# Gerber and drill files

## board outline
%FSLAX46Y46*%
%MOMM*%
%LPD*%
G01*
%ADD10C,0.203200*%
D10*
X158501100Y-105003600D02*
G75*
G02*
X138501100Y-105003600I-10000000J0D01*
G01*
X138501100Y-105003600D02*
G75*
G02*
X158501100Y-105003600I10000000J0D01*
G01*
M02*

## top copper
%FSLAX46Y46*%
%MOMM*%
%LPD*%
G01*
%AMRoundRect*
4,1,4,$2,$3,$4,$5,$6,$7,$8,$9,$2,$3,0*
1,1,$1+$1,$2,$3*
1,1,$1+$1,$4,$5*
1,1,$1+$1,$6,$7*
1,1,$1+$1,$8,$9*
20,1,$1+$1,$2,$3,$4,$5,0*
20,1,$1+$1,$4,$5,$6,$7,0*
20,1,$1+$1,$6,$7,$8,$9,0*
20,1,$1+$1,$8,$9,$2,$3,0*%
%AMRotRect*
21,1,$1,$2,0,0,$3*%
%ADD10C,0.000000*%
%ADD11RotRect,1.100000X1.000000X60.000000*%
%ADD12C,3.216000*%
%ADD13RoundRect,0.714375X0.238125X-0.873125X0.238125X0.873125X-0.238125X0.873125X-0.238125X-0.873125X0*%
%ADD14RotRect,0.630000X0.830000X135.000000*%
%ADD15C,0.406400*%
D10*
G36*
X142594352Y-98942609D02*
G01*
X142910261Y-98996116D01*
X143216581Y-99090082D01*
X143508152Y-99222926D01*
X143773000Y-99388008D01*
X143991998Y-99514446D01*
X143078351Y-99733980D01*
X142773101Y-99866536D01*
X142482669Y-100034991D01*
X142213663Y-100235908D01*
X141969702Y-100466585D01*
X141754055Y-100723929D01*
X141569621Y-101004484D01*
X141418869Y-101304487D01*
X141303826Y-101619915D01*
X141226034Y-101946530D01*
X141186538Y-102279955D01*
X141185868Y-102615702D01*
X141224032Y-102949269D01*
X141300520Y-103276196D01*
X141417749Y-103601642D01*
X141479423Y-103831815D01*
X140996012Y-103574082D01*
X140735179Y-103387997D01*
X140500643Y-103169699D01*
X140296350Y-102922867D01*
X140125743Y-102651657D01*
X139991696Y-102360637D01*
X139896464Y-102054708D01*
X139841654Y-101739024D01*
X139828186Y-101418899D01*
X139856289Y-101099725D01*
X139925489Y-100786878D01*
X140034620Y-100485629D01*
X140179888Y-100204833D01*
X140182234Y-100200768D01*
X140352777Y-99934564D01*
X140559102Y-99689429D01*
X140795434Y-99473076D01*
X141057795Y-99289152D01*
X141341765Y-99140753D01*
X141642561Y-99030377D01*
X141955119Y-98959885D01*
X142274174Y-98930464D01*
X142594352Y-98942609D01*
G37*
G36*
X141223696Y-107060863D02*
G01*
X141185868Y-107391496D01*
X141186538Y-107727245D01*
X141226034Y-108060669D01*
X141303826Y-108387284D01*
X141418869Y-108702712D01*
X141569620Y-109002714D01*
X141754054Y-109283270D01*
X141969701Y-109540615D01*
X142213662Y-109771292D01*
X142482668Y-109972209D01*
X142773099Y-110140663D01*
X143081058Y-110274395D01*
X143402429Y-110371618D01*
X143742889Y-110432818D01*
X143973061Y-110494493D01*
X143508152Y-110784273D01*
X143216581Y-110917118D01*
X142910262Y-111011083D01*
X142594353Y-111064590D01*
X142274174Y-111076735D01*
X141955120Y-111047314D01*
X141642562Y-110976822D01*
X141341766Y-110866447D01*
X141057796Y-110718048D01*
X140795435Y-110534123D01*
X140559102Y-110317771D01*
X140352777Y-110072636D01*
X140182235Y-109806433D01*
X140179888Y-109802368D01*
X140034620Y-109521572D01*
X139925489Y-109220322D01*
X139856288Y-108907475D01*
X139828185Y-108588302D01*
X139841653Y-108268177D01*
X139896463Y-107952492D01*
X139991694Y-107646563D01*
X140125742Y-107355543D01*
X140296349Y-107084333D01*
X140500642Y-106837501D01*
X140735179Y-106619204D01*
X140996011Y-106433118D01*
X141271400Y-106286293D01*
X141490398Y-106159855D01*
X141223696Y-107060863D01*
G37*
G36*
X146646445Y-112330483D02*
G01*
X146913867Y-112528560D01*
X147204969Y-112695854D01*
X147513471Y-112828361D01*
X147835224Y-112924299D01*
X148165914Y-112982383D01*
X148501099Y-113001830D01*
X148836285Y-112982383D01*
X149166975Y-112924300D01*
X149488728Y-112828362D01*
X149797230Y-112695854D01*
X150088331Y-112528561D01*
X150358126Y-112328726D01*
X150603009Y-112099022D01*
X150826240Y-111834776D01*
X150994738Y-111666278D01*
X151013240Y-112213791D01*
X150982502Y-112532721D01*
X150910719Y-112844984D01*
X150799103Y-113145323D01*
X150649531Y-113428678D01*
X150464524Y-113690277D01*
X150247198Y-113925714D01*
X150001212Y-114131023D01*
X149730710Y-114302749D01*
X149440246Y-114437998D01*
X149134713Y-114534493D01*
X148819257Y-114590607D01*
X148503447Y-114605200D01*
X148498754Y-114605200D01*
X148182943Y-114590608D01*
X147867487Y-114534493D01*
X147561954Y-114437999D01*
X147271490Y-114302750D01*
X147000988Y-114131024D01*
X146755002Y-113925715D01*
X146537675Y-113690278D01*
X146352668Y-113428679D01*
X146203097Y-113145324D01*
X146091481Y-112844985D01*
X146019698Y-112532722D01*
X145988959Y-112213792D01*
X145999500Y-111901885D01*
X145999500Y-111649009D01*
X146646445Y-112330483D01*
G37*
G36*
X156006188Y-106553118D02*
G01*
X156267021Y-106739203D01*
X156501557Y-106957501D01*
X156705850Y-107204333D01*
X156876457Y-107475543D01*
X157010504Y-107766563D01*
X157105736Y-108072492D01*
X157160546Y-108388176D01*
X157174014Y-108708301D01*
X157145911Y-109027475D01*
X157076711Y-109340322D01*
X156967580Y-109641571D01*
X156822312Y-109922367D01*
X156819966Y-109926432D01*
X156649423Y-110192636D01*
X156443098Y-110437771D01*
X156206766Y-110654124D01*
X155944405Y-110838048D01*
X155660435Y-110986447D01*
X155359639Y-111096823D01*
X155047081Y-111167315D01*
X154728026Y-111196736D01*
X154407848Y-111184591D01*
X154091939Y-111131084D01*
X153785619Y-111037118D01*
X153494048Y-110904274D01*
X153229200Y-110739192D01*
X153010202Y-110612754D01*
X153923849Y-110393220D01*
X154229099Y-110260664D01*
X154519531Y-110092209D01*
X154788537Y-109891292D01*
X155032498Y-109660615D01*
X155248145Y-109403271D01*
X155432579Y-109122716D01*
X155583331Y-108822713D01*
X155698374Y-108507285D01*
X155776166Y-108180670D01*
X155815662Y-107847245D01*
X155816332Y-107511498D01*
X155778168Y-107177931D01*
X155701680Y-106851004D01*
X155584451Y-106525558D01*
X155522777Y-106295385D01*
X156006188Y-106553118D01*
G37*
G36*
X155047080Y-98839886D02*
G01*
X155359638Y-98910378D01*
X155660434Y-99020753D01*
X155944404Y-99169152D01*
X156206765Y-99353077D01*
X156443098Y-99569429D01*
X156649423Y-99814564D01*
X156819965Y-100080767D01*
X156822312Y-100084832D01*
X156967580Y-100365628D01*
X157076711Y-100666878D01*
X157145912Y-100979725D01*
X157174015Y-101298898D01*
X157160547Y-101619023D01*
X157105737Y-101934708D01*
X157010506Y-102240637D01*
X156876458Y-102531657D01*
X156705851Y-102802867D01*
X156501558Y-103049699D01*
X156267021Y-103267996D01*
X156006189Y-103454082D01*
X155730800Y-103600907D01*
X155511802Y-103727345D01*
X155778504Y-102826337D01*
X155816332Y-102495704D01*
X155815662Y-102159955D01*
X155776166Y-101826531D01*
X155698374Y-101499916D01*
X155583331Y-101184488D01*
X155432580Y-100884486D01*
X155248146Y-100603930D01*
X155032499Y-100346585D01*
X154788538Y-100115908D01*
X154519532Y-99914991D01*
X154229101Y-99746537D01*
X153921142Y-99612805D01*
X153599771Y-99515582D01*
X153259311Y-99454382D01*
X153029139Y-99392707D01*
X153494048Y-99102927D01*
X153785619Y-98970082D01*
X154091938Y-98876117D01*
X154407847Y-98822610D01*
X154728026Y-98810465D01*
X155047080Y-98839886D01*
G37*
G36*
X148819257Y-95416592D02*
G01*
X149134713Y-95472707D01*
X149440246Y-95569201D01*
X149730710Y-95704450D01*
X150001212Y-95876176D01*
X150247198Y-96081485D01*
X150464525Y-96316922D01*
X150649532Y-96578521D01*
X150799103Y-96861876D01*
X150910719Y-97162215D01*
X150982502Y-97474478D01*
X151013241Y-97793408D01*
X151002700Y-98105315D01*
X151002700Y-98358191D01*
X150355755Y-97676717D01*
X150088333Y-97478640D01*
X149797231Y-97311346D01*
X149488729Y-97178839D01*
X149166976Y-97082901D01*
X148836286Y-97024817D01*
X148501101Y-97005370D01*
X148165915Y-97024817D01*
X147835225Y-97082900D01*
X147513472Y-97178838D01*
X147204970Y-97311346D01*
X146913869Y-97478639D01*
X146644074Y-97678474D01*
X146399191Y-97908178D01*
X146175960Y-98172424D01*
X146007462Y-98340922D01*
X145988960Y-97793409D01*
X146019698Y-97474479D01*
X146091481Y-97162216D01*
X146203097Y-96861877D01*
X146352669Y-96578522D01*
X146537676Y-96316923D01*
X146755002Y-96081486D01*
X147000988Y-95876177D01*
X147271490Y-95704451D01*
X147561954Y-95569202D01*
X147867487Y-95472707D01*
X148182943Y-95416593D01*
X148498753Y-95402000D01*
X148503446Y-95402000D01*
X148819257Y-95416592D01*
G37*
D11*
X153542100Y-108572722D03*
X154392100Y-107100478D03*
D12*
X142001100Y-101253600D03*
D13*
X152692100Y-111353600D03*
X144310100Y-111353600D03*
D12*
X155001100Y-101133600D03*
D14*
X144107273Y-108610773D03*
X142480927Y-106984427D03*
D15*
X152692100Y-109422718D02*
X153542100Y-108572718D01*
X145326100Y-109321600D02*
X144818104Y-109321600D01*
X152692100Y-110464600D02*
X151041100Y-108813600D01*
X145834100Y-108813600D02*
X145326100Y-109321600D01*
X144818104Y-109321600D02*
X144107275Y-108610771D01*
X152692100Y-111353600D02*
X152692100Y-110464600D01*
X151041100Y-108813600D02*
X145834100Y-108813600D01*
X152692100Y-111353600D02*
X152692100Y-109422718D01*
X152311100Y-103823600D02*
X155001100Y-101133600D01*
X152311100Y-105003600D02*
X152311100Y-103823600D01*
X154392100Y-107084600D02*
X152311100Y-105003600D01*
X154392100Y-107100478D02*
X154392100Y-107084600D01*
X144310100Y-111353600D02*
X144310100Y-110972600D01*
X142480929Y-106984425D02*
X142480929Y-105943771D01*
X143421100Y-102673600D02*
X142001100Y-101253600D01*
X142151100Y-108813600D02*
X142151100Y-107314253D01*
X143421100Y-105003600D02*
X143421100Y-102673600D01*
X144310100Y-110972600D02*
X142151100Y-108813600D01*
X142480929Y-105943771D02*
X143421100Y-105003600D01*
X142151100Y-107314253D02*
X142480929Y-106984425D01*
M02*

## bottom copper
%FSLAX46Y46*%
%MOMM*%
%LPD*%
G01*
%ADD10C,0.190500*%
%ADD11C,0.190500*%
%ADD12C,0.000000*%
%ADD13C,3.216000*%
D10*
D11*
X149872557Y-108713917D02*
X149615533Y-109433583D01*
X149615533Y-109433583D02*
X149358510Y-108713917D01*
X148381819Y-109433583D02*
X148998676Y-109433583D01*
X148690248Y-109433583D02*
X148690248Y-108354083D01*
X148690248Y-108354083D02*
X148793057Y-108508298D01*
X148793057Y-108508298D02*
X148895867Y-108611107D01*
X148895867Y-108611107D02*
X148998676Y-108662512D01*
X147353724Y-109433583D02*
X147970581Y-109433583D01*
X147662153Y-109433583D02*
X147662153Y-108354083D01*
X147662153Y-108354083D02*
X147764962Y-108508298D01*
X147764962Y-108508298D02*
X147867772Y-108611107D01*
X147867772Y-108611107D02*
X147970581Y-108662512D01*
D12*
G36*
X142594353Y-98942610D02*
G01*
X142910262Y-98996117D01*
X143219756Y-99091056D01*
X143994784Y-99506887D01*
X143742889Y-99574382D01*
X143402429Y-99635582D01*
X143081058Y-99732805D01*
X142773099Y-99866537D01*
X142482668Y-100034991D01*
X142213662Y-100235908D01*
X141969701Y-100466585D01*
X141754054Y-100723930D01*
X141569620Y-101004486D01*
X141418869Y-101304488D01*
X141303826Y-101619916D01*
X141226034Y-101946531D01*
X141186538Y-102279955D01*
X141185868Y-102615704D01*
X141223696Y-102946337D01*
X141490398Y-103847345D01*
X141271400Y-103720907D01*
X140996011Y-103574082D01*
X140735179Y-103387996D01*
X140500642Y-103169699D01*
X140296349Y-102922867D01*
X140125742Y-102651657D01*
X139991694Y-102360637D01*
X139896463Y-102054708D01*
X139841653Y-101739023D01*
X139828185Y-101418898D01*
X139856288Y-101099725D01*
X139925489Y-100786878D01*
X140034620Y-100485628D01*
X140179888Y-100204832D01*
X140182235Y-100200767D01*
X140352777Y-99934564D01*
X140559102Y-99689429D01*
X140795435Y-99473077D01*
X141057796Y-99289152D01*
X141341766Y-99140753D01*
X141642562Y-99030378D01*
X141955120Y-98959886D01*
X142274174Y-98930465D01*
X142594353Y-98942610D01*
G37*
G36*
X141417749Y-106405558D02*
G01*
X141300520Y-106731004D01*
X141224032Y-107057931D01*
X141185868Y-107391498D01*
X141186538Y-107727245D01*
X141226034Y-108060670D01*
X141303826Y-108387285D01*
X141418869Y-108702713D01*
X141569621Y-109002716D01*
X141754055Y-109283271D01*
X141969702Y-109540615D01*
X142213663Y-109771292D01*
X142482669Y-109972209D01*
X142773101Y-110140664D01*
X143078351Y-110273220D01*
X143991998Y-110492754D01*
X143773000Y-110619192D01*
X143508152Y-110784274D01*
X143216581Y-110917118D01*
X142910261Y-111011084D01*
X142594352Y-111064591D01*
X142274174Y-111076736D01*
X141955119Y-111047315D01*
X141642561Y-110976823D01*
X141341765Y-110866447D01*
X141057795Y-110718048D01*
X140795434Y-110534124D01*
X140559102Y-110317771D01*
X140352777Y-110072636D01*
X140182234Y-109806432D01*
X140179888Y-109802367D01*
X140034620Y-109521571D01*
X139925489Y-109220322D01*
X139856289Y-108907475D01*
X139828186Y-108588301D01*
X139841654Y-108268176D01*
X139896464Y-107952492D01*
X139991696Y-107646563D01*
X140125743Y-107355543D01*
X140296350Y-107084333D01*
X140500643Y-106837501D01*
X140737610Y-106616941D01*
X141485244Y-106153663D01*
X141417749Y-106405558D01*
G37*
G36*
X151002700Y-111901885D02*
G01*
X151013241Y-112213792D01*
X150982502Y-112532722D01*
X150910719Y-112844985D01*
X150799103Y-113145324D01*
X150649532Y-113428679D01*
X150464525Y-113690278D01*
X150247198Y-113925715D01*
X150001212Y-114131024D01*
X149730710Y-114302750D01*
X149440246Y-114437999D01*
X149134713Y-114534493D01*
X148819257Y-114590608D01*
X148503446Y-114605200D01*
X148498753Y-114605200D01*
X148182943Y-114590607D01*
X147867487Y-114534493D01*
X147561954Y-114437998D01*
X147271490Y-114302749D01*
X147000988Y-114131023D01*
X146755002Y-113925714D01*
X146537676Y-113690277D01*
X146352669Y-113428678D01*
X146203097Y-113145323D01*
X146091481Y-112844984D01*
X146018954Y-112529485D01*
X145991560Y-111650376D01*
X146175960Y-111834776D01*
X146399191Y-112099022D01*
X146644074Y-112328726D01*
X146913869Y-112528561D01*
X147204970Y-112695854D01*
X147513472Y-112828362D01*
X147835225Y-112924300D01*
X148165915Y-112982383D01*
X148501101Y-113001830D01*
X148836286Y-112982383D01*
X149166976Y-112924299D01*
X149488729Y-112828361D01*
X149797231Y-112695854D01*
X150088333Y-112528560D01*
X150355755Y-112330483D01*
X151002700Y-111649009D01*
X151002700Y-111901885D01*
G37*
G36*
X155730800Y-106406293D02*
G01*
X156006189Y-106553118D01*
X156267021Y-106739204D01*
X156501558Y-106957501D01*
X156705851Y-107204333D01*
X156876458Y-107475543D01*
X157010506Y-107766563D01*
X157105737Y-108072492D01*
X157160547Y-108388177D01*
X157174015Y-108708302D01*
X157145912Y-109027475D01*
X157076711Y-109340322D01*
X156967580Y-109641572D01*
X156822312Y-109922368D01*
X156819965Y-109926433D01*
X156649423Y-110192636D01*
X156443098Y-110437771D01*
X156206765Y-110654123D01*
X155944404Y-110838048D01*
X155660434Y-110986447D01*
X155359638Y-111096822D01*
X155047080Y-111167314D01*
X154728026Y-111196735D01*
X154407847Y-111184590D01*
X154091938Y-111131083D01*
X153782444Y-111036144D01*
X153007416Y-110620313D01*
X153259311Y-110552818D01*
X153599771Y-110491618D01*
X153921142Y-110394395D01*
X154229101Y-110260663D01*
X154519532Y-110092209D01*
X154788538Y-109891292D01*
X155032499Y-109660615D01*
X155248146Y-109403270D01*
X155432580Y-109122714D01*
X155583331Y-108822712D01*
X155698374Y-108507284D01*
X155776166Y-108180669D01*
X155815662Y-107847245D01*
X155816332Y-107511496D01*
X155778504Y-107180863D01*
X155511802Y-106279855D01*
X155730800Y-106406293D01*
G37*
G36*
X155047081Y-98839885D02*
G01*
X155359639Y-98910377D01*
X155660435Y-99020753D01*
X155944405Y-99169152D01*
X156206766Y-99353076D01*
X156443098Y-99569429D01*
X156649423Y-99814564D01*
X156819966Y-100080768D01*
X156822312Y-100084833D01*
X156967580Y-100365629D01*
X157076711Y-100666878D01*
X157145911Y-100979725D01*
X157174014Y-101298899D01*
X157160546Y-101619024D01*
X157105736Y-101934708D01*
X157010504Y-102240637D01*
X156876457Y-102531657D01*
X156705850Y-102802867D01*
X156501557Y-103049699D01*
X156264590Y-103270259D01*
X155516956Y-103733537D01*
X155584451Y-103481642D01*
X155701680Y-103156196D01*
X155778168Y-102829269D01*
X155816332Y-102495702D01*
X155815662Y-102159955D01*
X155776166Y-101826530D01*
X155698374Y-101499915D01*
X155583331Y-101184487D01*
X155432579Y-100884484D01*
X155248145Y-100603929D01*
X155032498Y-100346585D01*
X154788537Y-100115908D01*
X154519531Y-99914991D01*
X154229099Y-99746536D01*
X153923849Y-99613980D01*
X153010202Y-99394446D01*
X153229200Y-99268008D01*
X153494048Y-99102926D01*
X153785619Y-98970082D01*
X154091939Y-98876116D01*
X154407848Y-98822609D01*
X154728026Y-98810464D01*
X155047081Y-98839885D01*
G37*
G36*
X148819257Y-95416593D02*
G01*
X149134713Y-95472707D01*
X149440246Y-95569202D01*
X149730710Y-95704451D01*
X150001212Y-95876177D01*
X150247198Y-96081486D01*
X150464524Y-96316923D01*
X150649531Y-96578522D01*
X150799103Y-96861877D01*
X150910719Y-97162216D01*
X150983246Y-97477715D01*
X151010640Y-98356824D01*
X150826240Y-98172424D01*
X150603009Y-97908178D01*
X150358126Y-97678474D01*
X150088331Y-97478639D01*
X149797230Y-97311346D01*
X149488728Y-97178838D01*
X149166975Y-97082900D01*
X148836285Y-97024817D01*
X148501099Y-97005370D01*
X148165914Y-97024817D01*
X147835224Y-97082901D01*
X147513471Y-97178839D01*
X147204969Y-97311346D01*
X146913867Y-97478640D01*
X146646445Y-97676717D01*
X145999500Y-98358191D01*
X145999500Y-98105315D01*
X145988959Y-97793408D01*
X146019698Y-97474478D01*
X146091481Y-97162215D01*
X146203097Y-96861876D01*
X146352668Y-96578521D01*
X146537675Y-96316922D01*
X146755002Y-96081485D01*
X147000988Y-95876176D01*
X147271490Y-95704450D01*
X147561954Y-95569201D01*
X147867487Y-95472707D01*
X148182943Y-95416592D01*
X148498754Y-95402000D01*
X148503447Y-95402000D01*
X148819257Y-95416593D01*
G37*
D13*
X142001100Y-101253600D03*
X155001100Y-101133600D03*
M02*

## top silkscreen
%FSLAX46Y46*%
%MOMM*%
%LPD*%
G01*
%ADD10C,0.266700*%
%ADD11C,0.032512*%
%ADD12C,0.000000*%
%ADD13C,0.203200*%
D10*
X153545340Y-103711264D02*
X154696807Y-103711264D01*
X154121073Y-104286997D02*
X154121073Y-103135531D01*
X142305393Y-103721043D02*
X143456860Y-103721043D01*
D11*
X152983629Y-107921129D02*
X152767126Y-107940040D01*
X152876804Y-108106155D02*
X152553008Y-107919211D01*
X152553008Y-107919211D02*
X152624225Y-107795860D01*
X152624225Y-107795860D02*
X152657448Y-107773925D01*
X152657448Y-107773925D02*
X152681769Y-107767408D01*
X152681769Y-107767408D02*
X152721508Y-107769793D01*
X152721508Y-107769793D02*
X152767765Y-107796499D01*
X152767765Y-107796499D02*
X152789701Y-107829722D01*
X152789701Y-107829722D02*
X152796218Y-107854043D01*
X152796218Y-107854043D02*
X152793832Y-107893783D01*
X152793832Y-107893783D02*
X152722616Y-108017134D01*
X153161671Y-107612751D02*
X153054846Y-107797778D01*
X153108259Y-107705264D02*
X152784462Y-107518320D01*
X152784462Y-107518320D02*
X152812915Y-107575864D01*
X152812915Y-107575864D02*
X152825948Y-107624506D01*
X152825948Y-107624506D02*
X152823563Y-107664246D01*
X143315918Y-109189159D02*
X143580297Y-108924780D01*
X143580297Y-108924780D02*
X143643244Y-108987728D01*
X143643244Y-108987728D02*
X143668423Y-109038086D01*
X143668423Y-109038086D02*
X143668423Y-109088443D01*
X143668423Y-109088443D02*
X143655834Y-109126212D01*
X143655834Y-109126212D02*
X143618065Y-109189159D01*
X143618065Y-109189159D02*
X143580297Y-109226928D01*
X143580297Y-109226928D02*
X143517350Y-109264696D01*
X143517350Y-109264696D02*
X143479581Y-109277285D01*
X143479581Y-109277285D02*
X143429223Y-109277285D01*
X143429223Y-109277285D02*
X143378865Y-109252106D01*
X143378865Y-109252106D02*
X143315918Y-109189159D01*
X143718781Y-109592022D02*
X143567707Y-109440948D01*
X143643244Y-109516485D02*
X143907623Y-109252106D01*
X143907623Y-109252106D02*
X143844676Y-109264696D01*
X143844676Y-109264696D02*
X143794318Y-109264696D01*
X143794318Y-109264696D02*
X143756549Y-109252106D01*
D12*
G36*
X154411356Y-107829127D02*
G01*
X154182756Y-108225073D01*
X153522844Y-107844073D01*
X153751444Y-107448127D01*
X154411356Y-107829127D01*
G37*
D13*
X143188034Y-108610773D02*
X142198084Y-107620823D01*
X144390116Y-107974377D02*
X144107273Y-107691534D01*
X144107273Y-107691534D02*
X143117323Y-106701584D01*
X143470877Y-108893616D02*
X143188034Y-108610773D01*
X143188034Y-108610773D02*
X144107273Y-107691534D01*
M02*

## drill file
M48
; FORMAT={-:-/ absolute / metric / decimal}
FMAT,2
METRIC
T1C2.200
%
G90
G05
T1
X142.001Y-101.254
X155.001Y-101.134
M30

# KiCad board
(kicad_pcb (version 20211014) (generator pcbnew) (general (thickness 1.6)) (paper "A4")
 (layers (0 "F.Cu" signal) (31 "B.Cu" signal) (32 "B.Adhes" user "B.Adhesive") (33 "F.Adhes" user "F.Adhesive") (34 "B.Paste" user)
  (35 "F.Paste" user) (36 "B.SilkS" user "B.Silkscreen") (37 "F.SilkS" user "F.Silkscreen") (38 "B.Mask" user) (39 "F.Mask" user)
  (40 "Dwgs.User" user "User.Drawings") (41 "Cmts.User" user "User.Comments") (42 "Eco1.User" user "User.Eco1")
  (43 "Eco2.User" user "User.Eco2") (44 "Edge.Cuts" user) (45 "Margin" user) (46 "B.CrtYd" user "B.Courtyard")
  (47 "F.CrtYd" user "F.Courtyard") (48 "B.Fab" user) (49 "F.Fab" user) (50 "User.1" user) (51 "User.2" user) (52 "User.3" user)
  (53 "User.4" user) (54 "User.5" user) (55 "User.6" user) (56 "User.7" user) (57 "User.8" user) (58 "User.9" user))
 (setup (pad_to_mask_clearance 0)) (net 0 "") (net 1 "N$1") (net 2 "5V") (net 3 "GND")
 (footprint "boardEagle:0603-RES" (layer "F.Cu") (at 153.9671 107.8366 60)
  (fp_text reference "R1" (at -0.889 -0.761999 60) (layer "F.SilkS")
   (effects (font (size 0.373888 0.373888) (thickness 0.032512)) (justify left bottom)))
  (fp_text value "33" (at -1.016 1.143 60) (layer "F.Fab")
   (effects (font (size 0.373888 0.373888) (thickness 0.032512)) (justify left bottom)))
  (fp_poly (pts (xy -0.2286 0.381) (xy 0.2286 0.381) (xy 0.2286 -0.381) (xy -0.2286 -0.381)) (layer "F.SilkS") (width 0) (fill solid))
  (pad "1" smd rect (at -0.85 0 60) (size 1.1 1) (layers "F.Cu" "F.Paste" "F.Mask") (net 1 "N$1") (solder_mask_margin 0.1016))
  (pad "2" smd rect (at 0.85 0 60) (size 1.1 1) (layers "F.Cu" "F.Paste" "F.Mask") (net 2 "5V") (solder_mask_margin 0.1016)))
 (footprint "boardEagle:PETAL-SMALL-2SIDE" (layer "F.Cu") (at 142.0011 101.2536 -120)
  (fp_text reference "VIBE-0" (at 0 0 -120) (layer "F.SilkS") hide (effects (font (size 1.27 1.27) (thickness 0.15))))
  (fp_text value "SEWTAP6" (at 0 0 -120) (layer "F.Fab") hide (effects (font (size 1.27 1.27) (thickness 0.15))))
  (fp_poly
   (pts (xy -1.854655 -0.173117) (xy -1.587233 0.02496) (xy -1.296131 0.192254) (xy -0.987629 0.324761) (xy -0.665876 0.420699)
    (xy -0.335186 0.478783) (xy -0.000001 0.49823) (xy 0.335185 0.478783) (xy 0.665875 0.4207) (xy 0.987628 0.324762) (xy 1.29613 0.192254)
    (xy 1.587231 0.024961) (xy 1.857026 -0.174874) (xy 2.101909 -0.404578) (xy 2.32514 -0.668824) (xy 2.493638 -0.837322)
    (xy 2.51214 -0.289809) (xy 2.481402 0.029121) (xy 2.409619 0.341384) (xy 2.298003 0.641723) (xy 2.148431 0.925078)
    (xy 1.963424 1.186677) (xy 1.746098 1.422114) (xy 1.500112 1.627423) (xy 1.22961 1.799149) (xy 0.939146 1.934398) (xy 0.633613 2.030893)
    (xy 0.318157 2.087007) (xy 0.002347 2.1016) (xy -0.002346 2.1016) (xy -0.318157 2.087008) (xy -0.633613 2.030893)
    (xy -0.939146 1.934399) (xy -1.22961 1.79915) (xy -1.500112 1.627424) (xy -1.746098 1.422115) (xy -1.963425 1.186678)
    (xy -2.148432 0.925079) (xy -2.298003 0.641724) (xy -2.409619 0.341385) (xy -2.481402 0.029122) (xy -2.512141 -0.289808)
    (xy -2.5016 -0.601715) (xy -2.5016 -0.854591))
   (layer "F.Cu") (width 0) (fill solid))
  (fp_poly
   (pts (xy 2.5016 -0.601715) (xy 2.512141 -0.289808) (xy 2.481402 0.029122) (xy 2.409619 0.341385) (xy 2.298003 0.641724)
    (xy 2.148432 0.925079) (xy 1.963425 1.186678) (xy 1.746098 1.422115) (xy 1.500112 1.627424) (xy 1.22961 1.79915) (xy 0.939146 1.934399)
    (xy 0.633613 2.030893) (xy 0.318157 2.087008) (xy 0.002346 2.1016) (xy -0.002347 2.1016) (xy -0.318157 2.087007) (xy -0.633613 2.030893)
    (xy -0.939146 1.934398) (xy -1.22961 1.799149) (xy -1.500112 1.627423) (xy -1.746098 1.422114) (xy -1.963424 1.186677)
    (xy -2.148431 0.925078) (xy -2.298003 0.641723) (xy -2.409619 0.341384) (xy -2.482146 0.025885) (xy -2.50954 -0.853224)
    (xy -2.32514 -0.668824) (xy -2.101909 -0.404578) (xy -1.857026 -0.174874) (xy -1.587231 0.024961) (xy -1.29613 0.192254)
    (xy -0.987628 0.324762) (xy -0.665875 0.4207) (xy -0.335185 0.478783) (xy 0.000001 0.49823) (xy 0.335186 0.478783)
    (xy 0.665876 0.420699) (xy 0.987629 0.324761) (xy 1.296131 0.192254) (xy 1.587233 0.02496) (xy 1.854655 -0.173117) (xy 2.5016 -0.854591))
   (layer "B.Cu") (width 0) (fill solid))
  (pad "1" thru_hole circle (at 0 0 330) (size 3.216 3.216) (drill 2.2) (layers *.Cu *.Mask) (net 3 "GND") (solder_mask_margin 0.1016)))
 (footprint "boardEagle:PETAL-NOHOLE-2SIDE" (layer "F.Cu") (at 142.0011 108.7536 -60)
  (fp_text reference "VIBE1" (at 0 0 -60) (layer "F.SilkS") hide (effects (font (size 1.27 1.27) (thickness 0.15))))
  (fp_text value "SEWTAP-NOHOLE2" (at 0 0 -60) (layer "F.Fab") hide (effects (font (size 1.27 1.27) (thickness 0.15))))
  (fp_poly
   (pts (xy -1.854655 -0.173117) (xy -1.587233 0.02496) (xy -1.296131 0.192254) (xy -0.987629 0.324761) (xy -0.665876 0.420699)
    (xy -0.335186 0.478783) (xy -0.000001 0.49823) (xy 0.335185 0.478783) (xy 0.665875 0.4207) (xy 0.987628 0.324762) (xy 1.29613 0.192254)
    (xy 1.587231 0.024961) (xy 1.857026 -0.174874) (xy 2.101909 -0.404578) (xy 2.32514 -0.668824) (xy 2.493638 -0.837322)
    (xy 2.51214 -0.289809) (xy 2.481402 0.029121) (xy 2.409619 0.341384) (xy 2.298003 0.641723) (xy 2.148431 0.925078)
    (xy 1.963424 1.186677) (xy 1.746098 1.422114) (xy 1.500112 1.627423) (xy 1.22961 1.799149) (xy 0.939146 1.934398) (xy 0.633613 2.030893)
    (xy 0.318157 2.087007) (xy 0.002347 2.1016) (xy -0.002346 2.1016) (xy -0.318157 2.087008) (xy -0.633613 2.030893)
    (xy -0.939146 1.934399) (xy -1.22961 1.79915) (xy -1.500112 1.627424) (xy -1.746098 1.422115) (xy -1.963425 1.186678)
    (xy -2.148432 0.925079) (xy -2.298003 0.641724) (xy -2.409619 0.341385) (xy -2.481402 0.029122) (xy -2.512141 -0.289808)
    (xy -2.5016 -0.601715) (xy -2.5016 -0.854591))
   (layer "F.Cu") (width 0) (fill solid))
  (fp_poly
   (pts (xy 2.5016 -0.601715) (xy 2.512141 -0.289808) (xy 2.481402 0.029122) (xy 2.409619 0.341385) (xy 2.298003 0.641724)
    (xy 2.148432 0.925079) (xy 1.963425 1.186678) (xy 1.746098 1.422115) (xy 1.500112 1.627424) (xy 1.22961 1.79915) (xy 0.939146 1.934399)
    (xy 0.633613 2.030893) (xy 0.318157 2.087008) (xy 0.002346 2.1016) (xy -0.002347 2.1016) (xy -0.318157 2.087007) (xy -0.633613 2.030893)
    (xy -0.939146 1.934398) (xy -1.22961 1.799149) (xy -1.500112 1.627423) (xy -1.746098 1.422114) (xy -1.963424 1.186677)
    (xy -2.148431 0.925078) (xy -2.298003 0.641723) (xy -2.409619 0.341384) (xy -2.482146 0.025885) (xy -2.50954 -0.853224)
    (xy -2.32514 -0.668824) (xy -2.101909 -0.404578) (xy -1.857026 -0.174874) (xy -1.587231 0.024961) (xy -1.29613 0.192254)
    (xy -0.987628 0.324762) (xy -0.665875 0.4207) (xy -0.335185 0.478783) (xy 0.000001 0.49823) (xy 0.335186 0.478783)
    (xy 0.665876 0.420699) (xy 0.987629 0.324761) (xy 1.296131 0.192254) (xy 1.587233 0.02496) (xy 1.854655 -0.173117) (xy 2.5016 -0.854591))
   (layer "B.Cu") (width 0) (fill solid)))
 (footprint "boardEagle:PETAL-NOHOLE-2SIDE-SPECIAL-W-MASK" (layer "F.Cu") (at 148.5011 112.5036)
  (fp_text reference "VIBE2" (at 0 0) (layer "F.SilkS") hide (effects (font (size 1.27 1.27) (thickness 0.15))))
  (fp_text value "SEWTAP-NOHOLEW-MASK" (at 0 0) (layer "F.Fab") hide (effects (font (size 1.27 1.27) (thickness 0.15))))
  (fp_poly
   (pts (xy -1.854655 -0.173117) (xy -1.587233 0.02496) (xy -1.296131 0.192254) (xy -0.987629 0.324761) (xy -0.665876 0.420699)
    (xy -0.335186 0.478783) (xy -0.000001 0.49823) (xy 0.335185 0.478783) (xy 0.665875 0.4207) (xy 0.987628 0.324762) (xy 1.29613 0.192254)
    (xy 1.587231 0.024961) (xy 1.857026 -0.174874) (xy 2.101909 -0.404578) (xy 2.32514 -0.668824) (xy 2.493638 -0.837322)
    (xy 2.51214 -0.289809) (xy 2.481402 0.029121) (xy 2.409619 0.341384) (xy 2.298003 0.641723) (xy 2.148431 0.925078)
    (xy 1.963424 1.186677) (xy 1.746098 1.422114) (xy 1.500112 1.627423) (xy 1.22961 1.799149) (xy 0.939146 1.934398) (xy 0.633613 2.030893)
    (xy 0.318157 2.087007) (xy 0.002347 2.1016) (xy -0.002346 2.1016) (xy -0.318157 2.087008) (xy -0.633613 2.030893)
    (xy -0.939146 1.934399) (xy -1.22961 1.79915) (xy -1.500112 1.627424) (xy -1.746098 1.422115) (xy -1.963425 1.186678)
    (xy -2.148432 0.925079) (xy -2.298003 0.641724) (xy -2.409619 0.341385) (xy -2.481402 0.029122) (xy -2.512141 -0.289808)
    (xy -2.5016 -0.601715) (xy -2.5016 -0.854591))
   (layer "F.Cu") (width 0) (fill solid))
  (fp_poly
   (pts (xy 2.5016 -0.601715) (xy 2.512141 -0.289808) (xy 2.481402 0.029122) (xy 2.409619 0.341385) (xy 2.298003 0.641724)
    (xy 2.148432 0.925079) (xy 1.963425 1.186678) (xy 1.746098 1.422115) (xy 1.500112 1.627424) (xy 1.22961 1.79915) (xy 0.939146 1.934399)
    (xy 0.633613 2.030893) (xy 0.318157 2.087008) (xy 0.002346 2.1016) (xy -0.002347 2.1016) (xy -0.318157 2.087007) (xy -0.633613 2.030893)
    (xy -0.939146 1.934398) (xy -1.22961 1.799149) (xy -1.500112 1.627423) (xy -1.746098 1.422114) (xy -1.963424 1.186677)
    (xy -2.148431 0.925078) (xy -2.298003 0.641723) (xy -2.409619 0.341384) (xy -2.482146 0.025885) (xy -2.50954 -0.853224)
    (xy -2.32514 -0.668824) (xy -2.101909 -0.404578) (xy -1.857026 -0.174874) (xy -1.587231 0.024961) (xy -1.29613 0.192254)
    (xy -0.987628 0.324762) (xy -0.665875 0.4207) (xy -0.335185 0.478783) (xy 0.000001 0.49823) (xy 0.335186 0.478783)
    (xy 0.665876 0.420699) (xy 0.987629 0.324761) (xy 1.296131 0.192254) (xy 1.587233 0.02496) (xy 1.854655 -0.173117) (xy 2.5016 -0.854591))
   (layer "B.Cu") (width 0) (fill solid)))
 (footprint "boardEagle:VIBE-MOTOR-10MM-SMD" (layer "F.Cu") (at 148.5011 104.1146)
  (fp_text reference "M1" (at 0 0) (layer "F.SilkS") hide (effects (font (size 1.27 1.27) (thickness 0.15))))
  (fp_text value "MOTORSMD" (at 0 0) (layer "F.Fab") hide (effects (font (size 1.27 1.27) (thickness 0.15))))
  (pad "P$1" smd roundrect (at 4.191 7.239 90) (size 3.175 1.905) (layers "F.Cu" "F.Paste" "F.Mask") (roundrect_rratio 0.375) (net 1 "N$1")
   (solder_mask_margin 0.1016))
  (pad "P$2" smd roundrect (at -4.191 7.239 90) (size 3.175 1.905) (layers "F.Cu" "F.Paste" "F.Mask") (roundrect_rratio 0.375) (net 3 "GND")
   (solder_mask_margin 0.1016)))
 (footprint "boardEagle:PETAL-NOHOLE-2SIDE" (layer "F.Cu") (at 155.0011 108.8736 60)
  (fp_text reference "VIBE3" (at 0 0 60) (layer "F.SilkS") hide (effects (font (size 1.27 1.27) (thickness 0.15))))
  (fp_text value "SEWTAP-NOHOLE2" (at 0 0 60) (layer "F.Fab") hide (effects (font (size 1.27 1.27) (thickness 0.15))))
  (fp_poly
   (pts (xy -1.854655 -0.173117) (xy -1.587233 0.02496) (xy -1.296131 0.192254) (xy -0.987629 0.324761) (xy -0.665876 0.420699)
    (xy -0.335186 0.478783) (xy -0.000001 0.49823) (xy 0.335185 0.478783) (xy 0.665875 0.4207) (xy 0.987628 0.324762) (xy 1.29613 0.192254)
    (xy 1.587231 0.024961) (xy 1.857026 -0.174874) (xy 2.101909 -0.404578) (xy 2.32514 -0.668824) (xy 2.493638 -0.837322)
    (xy 2.51214 -0.289809) (xy 2.481402 0.029121) (xy 2.409619 0.341384) (xy 2.298003 0.641723) (xy 2.148431 0.925078)
    (xy 1.963424 1.186677) (xy 1.746098 1.422114) (xy 1.500112 1.627423) (xy 1.22961 1.799149) (xy 0.939146 1.934398) (xy 0.633613 2.030893)
    (xy 0.318157 2.087007) (xy 0.002347 2.1016) (xy -0.002346 2.1016) (xy -0.318157 2.087008) (xy -0.633613 2.030893)
    (xy -0.939146 1.934399) (xy -1.22961 1.79915) (xy -1.500112 1.627424) (xy -1.746098 1.422115) (xy -1.963425 1.186678)
    (xy -2.148432 0.925079) (xy -2.298003 0.641724) (xy -2.409619 0.341385) (xy -2.481402 0.029122) (xy -2.512141 -0.289808)
    (xy -2.5016 -0.601715) (xy -2.5016 -0.854591))
   (layer "F.Cu") (width 0) (fill solid))
  (fp_poly
   (pts (xy 2.5016 -0.601715) (xy 2.512141 -0.289808) (xy 2.481402 0.029122) (xy 2.409619 0.341385) (xy 2.298003 0.641724)
    (xy 2.148432 0.925079) (xy 1.963425 1.186678) (xy 1.746098 1.422115) (xy 1.500112 1.627424) (xy 1.22961 1.79915) (xy 0.939146 1.934399)
    (xy 0.633613 2.030893) (xy 0.318157 2.087008) (xy 0.002346 2.1016) (xy -0.002347 2.1016) (xy -0.318157 2.087007) (xy -0.633613 2.030893)
    (xy -0.939146 1.934398) (xy -1.22961 1.799149) (xy -1.500112 1.627423) (xy -1.746098 1.422114) (xy -1.963424 1.186677)
    (xy -2.148431 0.925078) (xy -2.298003 0.641723) (xy -2.409619 0.341384) (xy -2.482146 0.025885) (xy -2.50954 -0.853224)
    (xy -2.32514 -0.668824) (xy -2.101909 -0.404578) (xy -1.857026 -0.174874) (xy -1.587231 0.024961) (xy -1.29613 0.192254)
    (xy -0.987628 0.324762) (xy -0.665875 0.4207) (xy -0.335185 0.478783) (xy 0.000001 0.49823) (xy 0.335186 0.478783)
    (xy 0.665876 0.420699) (xy 0.987629 0.324761) (xy 1.296131 0.192254) (xy 1.587233 0.02496) (xy 1.854655 -0.173117) (xy 2.5016 -0.854591))
   (layer "B.Cu") (width 0) (fill solid)))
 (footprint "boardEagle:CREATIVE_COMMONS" (layer "F.Cu") (at 49.620044 105.0036)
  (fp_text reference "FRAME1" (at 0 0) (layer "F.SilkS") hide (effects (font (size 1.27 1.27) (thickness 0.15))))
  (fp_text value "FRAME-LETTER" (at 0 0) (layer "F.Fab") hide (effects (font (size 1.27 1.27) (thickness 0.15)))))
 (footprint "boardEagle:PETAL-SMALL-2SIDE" (layer "F.Cu") (at 155.0011 101.1336 120)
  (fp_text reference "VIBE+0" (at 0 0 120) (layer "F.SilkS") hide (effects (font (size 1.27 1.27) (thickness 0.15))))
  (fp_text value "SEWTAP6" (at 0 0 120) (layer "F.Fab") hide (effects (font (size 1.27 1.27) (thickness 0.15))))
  (fp_poly
   (pts (xy -1.854655 -0.173117) (xy -1.587233 0.02496) (xy -1.296131 0.192254) (xy -0.987629 0.324761) (xy -0.665876 0.420699)
    (xy -0.335186 0.478783) (xy -0.000001 0.49823) (xy 0.335185 0.478783) (xy 0.665875 0.4207) (xy 0.987628 0.324762) (xy 1.29613 0.192254)
    (xy 1.587231 0.024961) (xy 1.857026 -0.174874) (xy 2.101909 -0.404578) (xy 2.32514 -0.668824) (xy 2.493638 -0.837322)
    (xy 2.51214 -0.289809) (xy 2.481402 0.029121) (xy 2.409619 0.341384) (xy 2.298003 0.641723) (xy 2.148431 0.925078)
    (xy 1.963424 1.186677) (xy 1.746098 1.422114) (xy 1.500112 1.627423) (xy 1.22961 1.799149) (xy 0.939146 1.934398) (xy 0.633613 2.030893)
    (xy 0.318157 2.087007) (xy 0.002347 2.1016) (xy -0.002346 2.1016) (xy -0.318157 2.087008) (xy -0.633613 2.030893)
    (xy -0.939146 1.934399) (xy -1.22961 1.79915) (xy -1.500112 1.627424) (xy -1.746098 1.422115) (xy -1.963425 1.186678)
    (xy -2.148432 0.925079) (xy -2.298003 0.641724) (xy -2.409619 0.341385) (xy -2.481402 0.029122) (xy -2.512141 -0.289808)
    (xy -2.5016 -0.601715) (xy -2.5016 -0.854591))
   (layer "F.Cu") (width 0) (fill solid))
  (fp_poly
   (pts (xy 2.5016 -0.601715) (xy 2.512141 -0.289808) (xy 2.481402 0.029122) (xy 2.409619 0.341385) (xy 2.298003 0.641724)
    (xy 2.148432 0.925079) (xy 1.963425 1.186678) (xy 1.746098 1.422115) (xy 1.500112 1.627424) (xy 1.22961 1.79915) (xy 0.939146 1.934399)
    (xy 0.633613 2.030893) (xy 0.318157 2.087008) (xy 0.002346 2.1016) (xy -0.002347 2.1016) (xy -0.318157 2.087007) (xy -0.633613 2.030893)
    (xy -0.939146 1.934398) (xy -1.22961 1.799149) (xy -1.500112 1.627423) (xy -1.746098 1.422114) (xy -1.963424 1.186677)
    (xy -2.148431 0.925078) (xy -2.298003 0.641723) (xy -2.409619 0.341384) (xy -2.482146 0.025885) (xy -2.50954 -0.853224)
    (xy -2.32514 -0.668824) (xy -2.101909 -0.404578) (xy -1.857026 -0.174874) (xy -1.587231 0.024961) (xy -1.29613 0.192254)
    (xy -0.987628 0.324762) (xy -0.665875 0.4207) (xy -0.335185 0.478783) (xy 0.000001 0.49823) (xy 0.335186 0.478783)
    (xy 0.665876 0.420699) (xy 0.987629 0.324761) (xy 1.296131 0.192254) (xy 1.587233 0.02496) (xy 1.854655 -0.173117) (xy 2.5016 -0.854591))
   (layer "B.Cu") (width 0) (fill solid))
  (pad "1" thru_hole circle (at 0 0 210) (size 3.216 3.216) (drill 2.2) (layers *.Cu *.Mask) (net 2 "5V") (solder_mask_margin 0.1016)))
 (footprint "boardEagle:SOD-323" (layer "F.Cu") (at 143.2941 107.7976 135)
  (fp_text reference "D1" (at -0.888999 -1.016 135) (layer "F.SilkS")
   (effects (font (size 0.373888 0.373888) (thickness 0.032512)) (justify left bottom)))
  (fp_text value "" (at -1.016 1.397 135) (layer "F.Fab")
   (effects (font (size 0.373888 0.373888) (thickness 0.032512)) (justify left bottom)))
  (fp_line (start -0.5 -0.65) (end 0.9 -0.65) (layer "F.SilkS") (width 0.2032))
  (fp_line (start -0.9 0.65) (end -0.5 0.65) (layer "F.SilkS") (width 0.2032))
  (fp_line (start -0.5 0.65) (end 0.9 0.65) (layer "F.SilkS") (width 0.2032))
  (fp_line (start -0.9 -0.65) (end -0.5 -0.65) (layer "F.SilkS") (width 0.2032))
  (fp_line (start -0.5 -0.65) (end -0.5 0.65) (layer "F.SilkS") (width 0.2032))
  (pad "1" smd rect (at -1.15 0 135) (size 0.63 0.83) (layers "F.Cu" "F.Paste" "F.Mask") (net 1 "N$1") (solder_mask_margin 0.1016))
  (pad "2" smd rect (at 1.15 0 135) (size 0.63 0.83) (layers "F.Cu" "F.Paste" "F.Mask") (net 3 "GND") (solder_mask_margin 0.1016)))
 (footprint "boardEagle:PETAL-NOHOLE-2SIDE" (layer "F.Cu") (at 148.5011 97.5036 180)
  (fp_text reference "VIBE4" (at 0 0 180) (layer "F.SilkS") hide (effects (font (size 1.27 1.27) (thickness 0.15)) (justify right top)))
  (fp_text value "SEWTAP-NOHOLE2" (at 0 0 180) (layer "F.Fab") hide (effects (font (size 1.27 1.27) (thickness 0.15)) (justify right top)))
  (fp_poly
   (pts (xy -1.854655 -0.173117) (xy -1.587233 0.02496) (xy -1.296131 0.192254) (xy -0.987629 0.324761) (xy -0.665876 0.420699)
    (xy -0.335186 0.478783) (xy -0.000001 0.49823) (xy 0.335185 0.478783) (xy 0.665875 0.4207) (xy 0.987628 0.324762) (xy 1.29613 0.192254)
    (xy 1.587231 0.024961) (xy 1.857026 -0.174874) (xy 2.101909 -0.404578) (xy 2.32514 -0.668824) (xy 2.493638 -0.837322)
    (xy 2.51214 -0.289809) (xy 2.481402 0.029121) (xy 2.409619 0.341384) (xy 2.298003 0.641723) (xy 2.148431 0.925078)
    (xy 1.963424 1.186677) (xy 1.746098 1.422114) (xy 1.500112 1.627423) (xy 1.22961 1.799149) (xy 0.939146 1.934398) (xy 0.633613 2.030893)
    (xy 0.318157 2.087007) (xy 0.002347 2.1016) (xy -0.002346 2.1016) (xy -0.318157 2.087008) (xy -0.633613 2.030893)
    (xy -0.939146 1.934399) (xy -1.22961 1.79915) (xy -1.500112 1.627424) (xy -1.746098 1.422115) (xy -1.963425 1.186678)
    (xy -2.148432 0.925079) (xy -2.298003 0.641724) (xy -2.409619 0.341385) (xy -2.481402 0.029122) (xy -2.512141 -0.289808)
    (xy -2.5016 -0.601715) (xy -2.5016 -0.854591))
   (layer "F.Cu") (width 0) (fill solid))
  (fp_poly
   (pts (xy 2.5016 -0.601715) (xy 2.512141 -0.289808) (xy 2.481402 0.029122) (xy 2.409619 0.341385) (xy 2.298003 0.641724)
    (xy 2.148432 0.925079) (xy 1.963425 1.186678) (xy 1.746098 1.422115) (xy 1.500112 1.627424) (xy 1.22961 1.79915) (xy 0.939146 1.934399)
    (xy 0.633613 2.030893) (xy 0.318157 2.087008) (xy 0.002346 2.1016) (xy -0.002347 2.1016) (xy -0.318157 2.087007) (xy -0.633613 2.030893)
    (xy -0.939146 1.934398) (xy -1.22961 1.799149) (xy -1.500112 1.627423) (xy -1.746098 1.422114) (xy -1.963424 1.186677)
    (xy -2.148431 0.925078) (xy -2.298003 0.641723) (xy -2.409619 0.341384) (xy -2.482146 0.025885) (xy -2.50954 -0.853224)
    (xy -2.32514 -0.668824) (xy -2.101909 -0.404578) (xy -1.857026 -0.174874) (xy -1.587231 0.024961) (xy -1.29613 0.192254)
    (xy -0.987628 0.324762) (xy -0.665875 0.4207) (xy -0.335185 0.478783) (xy 0.000001 0.49823) (xy 0.335186 0.478783)
    (xy 0.665876 0.420699) (xy 0.987629 0.324761) (xy 1.296131 0.192254) (xy 1.587233 0.02496) (xy 1.854655 -0.173117) (xy 2.5016 -0.854591))
   (layer "B.Cu") (width 0) (fill solid)))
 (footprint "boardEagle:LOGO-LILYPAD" (layer "B.Cu") (at 148.5011 105.0036 180)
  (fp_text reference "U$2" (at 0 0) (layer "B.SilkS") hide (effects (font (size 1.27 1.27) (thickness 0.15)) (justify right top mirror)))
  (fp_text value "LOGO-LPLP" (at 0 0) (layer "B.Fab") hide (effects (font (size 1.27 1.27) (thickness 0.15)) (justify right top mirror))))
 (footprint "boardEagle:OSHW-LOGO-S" (layer "B.Cu") (at 148.5011 101.1936 180)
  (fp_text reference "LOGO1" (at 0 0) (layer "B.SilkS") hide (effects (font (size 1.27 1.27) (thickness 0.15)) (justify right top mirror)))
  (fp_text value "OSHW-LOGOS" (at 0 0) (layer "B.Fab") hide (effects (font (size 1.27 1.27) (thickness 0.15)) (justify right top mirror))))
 (gr_circle (center 148.5011 105.0036) (end 158.5011 105.0036) (layer "Edge.Cuts") (width 0.2032) (fill none))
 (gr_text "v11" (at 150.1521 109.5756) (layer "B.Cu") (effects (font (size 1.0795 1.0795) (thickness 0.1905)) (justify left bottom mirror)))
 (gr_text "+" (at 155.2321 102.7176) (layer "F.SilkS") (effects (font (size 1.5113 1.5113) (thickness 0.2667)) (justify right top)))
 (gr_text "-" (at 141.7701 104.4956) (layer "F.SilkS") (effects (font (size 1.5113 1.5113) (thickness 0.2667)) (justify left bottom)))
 (segment (start 152.6921 109.422718) (end 153.5421 108.572718) (width 0.4064) (layer "F.Cu") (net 1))
 (segment (start 145.3261 109.3216) (end 144.818104 109.3216) (width 0.4064) (layer "F.Cu") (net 1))
 (segment (start 152.6921 110.4646) (end 151.0411 108.8136) (width 0.4064) (layer "F.Cu") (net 1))
 (segment (start 145.8341 108.8136) (end 145.3261 109.3216) (width 0.4064) (layer "F.Cu") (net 1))
 (segment (start 144.818104 109.3216) (end 144.107275 108.610771) (width 0.4064) (layer "F.Cu") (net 1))
 (segment (start 152.6921 111.3536) (end 152.6921 110.4646) (width 0.4064) (layer "F.Cu") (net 1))
 (segment (start 151.0411 108.8136) (end 145.8341 108.8136) (width 0.4064) (layer "F.Cu") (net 1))
 (segment (start 152.6921 111.3536) (end 152.6921 109.422718) (width 0.4064) (layer "F.Cu") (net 1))
 (segment (start 152.3111 103.8236) (end 155.0011 101.1336) (width 0.4064) (layer "F.Cu") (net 2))
 (segment (start 152.3111 105.0036) (end 152.3111 103.8236) (width 0.4064) (layer "F.Cu") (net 2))
 (segment (start 154.3921 107.0846) (end 152.3111 105.0036) (width 0.4064) (layer "F.Cu") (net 2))
 (segment (start 154.3921 107.100478) (end 154.3921 107.0846) (width 0.4064) (layer "F.Cu") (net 2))
 (segment (start 144.3101 111.3536) (end 144.3101 110.9726) (width 0.4064) (layer "F.Cu") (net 3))
 (segment (start 142.480929 106.984425) (end 142.480929 105.943771) (width 0.4064) (layer "F.Cu") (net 3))
 (segment (start 143.4211 102.6736) (end 142.0011 101.2536) (width 0.4064) (layer "F.Cu") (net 3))
 (segment (start 142.1511 108.8136) (end 142.1511 107.314253) (width 0.4064) (layer "F.Cu") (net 3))
 (segment (start 143.4211 105.0036) (end 143.4211 102.6736) (width 0.4064) (layer "F.Cu") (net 3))
 (segment (start 144.3101 110.9726) (end 142.1511 108.8136) (width 0.4064) (layer "F.Cu") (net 3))
 (segment (start 142.480929 105.943771) (end 143.4211 105.0036) (width 0.4064) (layer "F.Cu") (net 3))
 (segment (start 142.1511 107.314253) (end 142.480929 106.984425) (width 0.4064) (layer "F.Cu") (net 3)))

